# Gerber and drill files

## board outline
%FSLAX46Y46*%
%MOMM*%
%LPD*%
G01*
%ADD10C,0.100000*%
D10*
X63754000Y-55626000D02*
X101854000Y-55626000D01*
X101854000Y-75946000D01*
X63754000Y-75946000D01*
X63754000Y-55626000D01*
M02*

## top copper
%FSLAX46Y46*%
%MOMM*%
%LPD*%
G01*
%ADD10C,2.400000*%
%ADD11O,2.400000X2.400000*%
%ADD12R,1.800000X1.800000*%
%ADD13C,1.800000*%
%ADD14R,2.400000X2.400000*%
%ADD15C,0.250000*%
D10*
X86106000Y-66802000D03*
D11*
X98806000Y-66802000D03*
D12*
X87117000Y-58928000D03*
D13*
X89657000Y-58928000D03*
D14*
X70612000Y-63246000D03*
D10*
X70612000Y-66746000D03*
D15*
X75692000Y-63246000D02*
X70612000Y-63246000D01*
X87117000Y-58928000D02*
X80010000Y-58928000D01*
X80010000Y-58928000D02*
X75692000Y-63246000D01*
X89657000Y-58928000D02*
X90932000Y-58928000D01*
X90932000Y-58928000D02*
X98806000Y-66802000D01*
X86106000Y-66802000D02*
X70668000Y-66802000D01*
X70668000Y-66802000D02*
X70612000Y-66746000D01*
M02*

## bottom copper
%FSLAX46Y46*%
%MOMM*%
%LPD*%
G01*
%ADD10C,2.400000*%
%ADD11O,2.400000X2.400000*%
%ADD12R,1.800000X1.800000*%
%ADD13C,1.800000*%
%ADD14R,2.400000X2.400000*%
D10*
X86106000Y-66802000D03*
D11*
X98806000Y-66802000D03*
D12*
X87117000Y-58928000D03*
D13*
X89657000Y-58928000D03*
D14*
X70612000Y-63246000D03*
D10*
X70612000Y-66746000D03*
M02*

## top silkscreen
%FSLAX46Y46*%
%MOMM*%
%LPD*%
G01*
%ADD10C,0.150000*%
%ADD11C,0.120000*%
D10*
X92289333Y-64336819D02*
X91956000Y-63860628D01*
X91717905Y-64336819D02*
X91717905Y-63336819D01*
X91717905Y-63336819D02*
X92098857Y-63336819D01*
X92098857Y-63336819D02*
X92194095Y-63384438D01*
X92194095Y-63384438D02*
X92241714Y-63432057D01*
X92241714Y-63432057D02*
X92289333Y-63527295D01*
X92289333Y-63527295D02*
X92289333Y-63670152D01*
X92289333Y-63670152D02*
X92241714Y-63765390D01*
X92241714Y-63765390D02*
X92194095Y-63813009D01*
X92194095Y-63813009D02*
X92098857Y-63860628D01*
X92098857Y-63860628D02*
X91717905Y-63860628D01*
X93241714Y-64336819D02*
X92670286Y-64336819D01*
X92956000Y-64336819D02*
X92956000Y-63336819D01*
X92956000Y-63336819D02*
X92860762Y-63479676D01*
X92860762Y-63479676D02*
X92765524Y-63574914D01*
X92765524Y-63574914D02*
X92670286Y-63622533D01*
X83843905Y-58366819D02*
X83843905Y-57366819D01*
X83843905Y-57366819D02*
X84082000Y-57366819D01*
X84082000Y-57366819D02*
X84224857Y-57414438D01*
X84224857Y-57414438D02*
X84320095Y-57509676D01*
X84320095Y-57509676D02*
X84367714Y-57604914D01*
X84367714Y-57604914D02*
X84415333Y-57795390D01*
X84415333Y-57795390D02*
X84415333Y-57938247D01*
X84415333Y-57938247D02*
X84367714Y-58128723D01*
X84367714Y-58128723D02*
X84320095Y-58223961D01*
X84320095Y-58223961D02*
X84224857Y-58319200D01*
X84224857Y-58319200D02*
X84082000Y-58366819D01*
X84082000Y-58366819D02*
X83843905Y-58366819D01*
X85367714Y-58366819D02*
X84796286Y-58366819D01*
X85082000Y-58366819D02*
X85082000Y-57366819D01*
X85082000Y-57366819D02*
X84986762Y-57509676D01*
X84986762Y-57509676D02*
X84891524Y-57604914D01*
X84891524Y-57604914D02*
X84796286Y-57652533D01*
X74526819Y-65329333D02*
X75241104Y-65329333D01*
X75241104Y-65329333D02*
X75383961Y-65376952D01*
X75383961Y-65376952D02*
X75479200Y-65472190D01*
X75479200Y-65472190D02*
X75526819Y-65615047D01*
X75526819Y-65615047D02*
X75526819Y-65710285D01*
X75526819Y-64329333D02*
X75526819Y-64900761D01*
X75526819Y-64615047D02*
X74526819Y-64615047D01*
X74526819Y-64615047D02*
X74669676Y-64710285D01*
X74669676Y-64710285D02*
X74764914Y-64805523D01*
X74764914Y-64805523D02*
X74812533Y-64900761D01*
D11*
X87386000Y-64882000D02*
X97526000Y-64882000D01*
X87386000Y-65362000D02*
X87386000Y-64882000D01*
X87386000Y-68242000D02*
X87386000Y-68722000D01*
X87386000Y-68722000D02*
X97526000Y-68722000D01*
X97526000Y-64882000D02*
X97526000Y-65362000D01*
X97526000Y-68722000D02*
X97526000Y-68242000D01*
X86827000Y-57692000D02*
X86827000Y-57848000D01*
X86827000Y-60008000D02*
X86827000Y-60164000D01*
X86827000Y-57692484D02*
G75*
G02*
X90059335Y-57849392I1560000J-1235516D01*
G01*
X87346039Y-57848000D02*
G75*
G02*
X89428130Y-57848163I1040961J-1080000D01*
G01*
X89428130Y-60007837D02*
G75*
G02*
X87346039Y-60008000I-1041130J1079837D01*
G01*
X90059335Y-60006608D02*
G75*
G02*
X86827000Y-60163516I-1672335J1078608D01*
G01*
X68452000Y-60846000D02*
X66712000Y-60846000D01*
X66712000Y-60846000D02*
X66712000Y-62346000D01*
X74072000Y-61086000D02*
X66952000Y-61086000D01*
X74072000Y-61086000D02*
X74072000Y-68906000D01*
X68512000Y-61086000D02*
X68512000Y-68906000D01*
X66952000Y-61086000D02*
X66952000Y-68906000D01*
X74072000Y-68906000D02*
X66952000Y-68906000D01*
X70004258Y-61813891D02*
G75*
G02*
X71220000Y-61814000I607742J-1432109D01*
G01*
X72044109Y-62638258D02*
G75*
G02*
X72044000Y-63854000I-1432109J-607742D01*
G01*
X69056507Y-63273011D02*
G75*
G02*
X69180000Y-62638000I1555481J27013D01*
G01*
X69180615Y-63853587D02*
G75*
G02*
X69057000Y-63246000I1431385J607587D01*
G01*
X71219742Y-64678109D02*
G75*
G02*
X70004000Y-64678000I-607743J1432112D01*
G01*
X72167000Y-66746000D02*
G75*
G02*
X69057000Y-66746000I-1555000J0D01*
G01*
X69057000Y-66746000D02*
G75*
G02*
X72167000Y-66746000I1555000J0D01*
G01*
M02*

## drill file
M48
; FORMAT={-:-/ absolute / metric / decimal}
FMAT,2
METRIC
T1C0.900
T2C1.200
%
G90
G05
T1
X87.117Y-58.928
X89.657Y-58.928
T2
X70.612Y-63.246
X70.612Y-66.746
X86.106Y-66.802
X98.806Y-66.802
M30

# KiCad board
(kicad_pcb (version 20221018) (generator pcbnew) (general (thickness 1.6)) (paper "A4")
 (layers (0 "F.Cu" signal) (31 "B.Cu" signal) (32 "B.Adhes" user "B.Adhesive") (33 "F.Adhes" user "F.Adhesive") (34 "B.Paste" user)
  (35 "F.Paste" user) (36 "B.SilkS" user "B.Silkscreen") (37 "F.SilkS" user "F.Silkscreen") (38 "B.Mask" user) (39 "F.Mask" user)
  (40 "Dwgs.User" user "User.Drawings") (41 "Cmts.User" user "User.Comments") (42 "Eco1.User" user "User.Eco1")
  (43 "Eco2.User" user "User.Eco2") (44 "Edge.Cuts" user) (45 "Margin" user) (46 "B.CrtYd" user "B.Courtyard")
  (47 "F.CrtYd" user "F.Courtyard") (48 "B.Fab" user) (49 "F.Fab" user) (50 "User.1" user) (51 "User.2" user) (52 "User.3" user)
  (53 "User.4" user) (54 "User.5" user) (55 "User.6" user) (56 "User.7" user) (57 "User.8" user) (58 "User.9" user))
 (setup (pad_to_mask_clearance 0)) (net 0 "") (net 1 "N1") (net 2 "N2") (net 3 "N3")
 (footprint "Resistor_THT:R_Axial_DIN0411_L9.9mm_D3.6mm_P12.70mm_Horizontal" (layer "F.Cu") (at 86.106 66.802)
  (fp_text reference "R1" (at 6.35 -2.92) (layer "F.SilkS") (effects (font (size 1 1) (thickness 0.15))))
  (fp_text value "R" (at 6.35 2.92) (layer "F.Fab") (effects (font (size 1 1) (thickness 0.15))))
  (fp_line (start 1.28 -1.92) (end 11.42 -1.92) (stroke (width 0.12) (type solid)) (layer "F.SilkS"))
  (fp_line (start 1.28 -1.44) (end 1.28 -1.92) (stroke (width 0.12) (type solid)) (layer "F.SilkS"))
  (fp_line (start 1.28 1.44) (end 1.28 1.92) (stroke (width 0.12) (type solid)) (layer "F.SilkS"))
  (fp_line (start 1.28 1.92) (end 11.42 1.92) (stroke (width 0.12) (type solid)) (layer "F.SilkS"))
  (fp_line (start 11.42 -1.92) (end 11.42 -1.44) (stroke (width 0.12) (type solid)) (layer "F.SilkS"))
  (fp_line (start 11.42 1.92) (end 11.42 1.44) (stroke (width 0.12) (type solid)) (layer "F.SilkS"))
  (pad "1" thru_hole circle (at 0 0) (size 2.4 2.4) (drill 1.2) (layers "*.Cu" "*.Mask") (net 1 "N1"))
  (pad "2" thru_hole oval (at 12.7 0) (size 2.4 2.4) (drill 1.2) (layers "*.Cu" "*.Mask") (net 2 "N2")))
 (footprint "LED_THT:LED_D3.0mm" (layer "F.Cu") (at 87.117 58.928)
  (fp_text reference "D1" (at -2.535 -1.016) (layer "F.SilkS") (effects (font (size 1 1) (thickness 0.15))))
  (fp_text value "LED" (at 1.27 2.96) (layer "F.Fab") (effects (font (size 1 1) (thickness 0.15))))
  (fp_line (start -0.29 -1.236) (end -0.29 -1.08) (stroke (width 0.12) (type solid)) (layer "F.SilkS"))
  (fp_line (start -0.29 1.08) (end -0.29 1.236) (stroke (width 0.12) (type solid)) (layer "F.SilkS"))
  (fp_arc (start -0.29 -1.235516) (mid 1.366487 -1.987659) (end 2.942335 -1.078608) (stroke (width 0.12) (type solid)) (layer "F.SilkS"))
  (fp_arc (start 0.229039 -1.08) (mid 1.270117 -1.5) (end 2.31113 -1.079837) (stroke (width 0.12) (type solid)) (layer "F.SilkS"))
  (fp_arc (start 2.31113 1.079837) (mid 1.270117 1.5) (end 0.229039 1.08) (stroke (width 0.12) (type solid)) (layer "F.SilkS"))
  (fp_arc (start 2.942335 1.078608) (mid 1.366487 1.987659) (end -0.29 1.235516) (stroke (width 0.12) (type solid)) (layer "F.SilkS"))
  (pad "1" thru_hole rect (at 0 0) (size 1.8 1.8) (drill 0.9) (layers "*.Cu" "*.Mask") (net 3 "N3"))
  (pad "2" thru_hole circle (at 2.54 0) (size 1.8 1.8) (drill 0.9) (layers "*.Cu" "*.Mask") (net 2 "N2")))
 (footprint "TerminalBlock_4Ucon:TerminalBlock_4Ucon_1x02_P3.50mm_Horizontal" (layer "F.Cu") (at 70.612 63.246 -90)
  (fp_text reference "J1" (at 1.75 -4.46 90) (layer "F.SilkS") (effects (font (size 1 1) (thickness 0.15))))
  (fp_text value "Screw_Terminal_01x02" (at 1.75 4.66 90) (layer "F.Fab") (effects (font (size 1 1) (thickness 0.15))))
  (fp_line (start -2.4 2.16) (end -2.4 3.9) (stroke (width 0.12) (type solid)) (layer "F.SilkS"))
  (fp_line (start -2.4 3.9) (end -0.9 3.9) (stroke (width 0.12) (type solid)) (layer "F.SilkS"))
  (fp_line (start -2.16 -3.46) (end -2.16 3.66) (stroke (width 0.12) (type solid)) (layer "F.SilkS"))
  (fp_line (start -2.16 -3.46) (end 5.66 -3.46) (stroke (width 0.12) (type solid)) (layer "F.SilkS"))
  (fp_line (start -2.16 2.1) (end 5.66 2.1) (stroke (width 0.12) (type solid)) (layer "F.SilkS"))
  (fp_line (start -2.16 3.66) (end 5.66 3.66) (stroke (width 0.12) (type solid)) (layer "F.SilkS"))
  (fp_line (start 5.66 -3.46) (end 5.66 3.66) (stroke (width 0.12) (type solid)) (layer "F.SilkS"))
  (fp_arc (start -1.432109 0.607742) (mid -1.555727 -0.00014) (end -1.432 -0.608) (stroke (width 0.12) (type solid)) (layer "F.SilkS"))
  (fp_arc (start -0.607742 -1.432109) (mid 0.00014 -1.555727) (end 0.608 -1.432) (stroke (width 0.12) (type solid)) (layer "F.SilkS"))
  (fp_arc (start 0.027011 1.555493) (mid -0.296984 1.527118) (end -0.608 1.432) (stroke (width 0.12) (type solid)) (layer "F.SilkS"))
  (fp_arc (start 0.607587 1.431385) (mid 0.310017 1.523783) (end 0 1.555) (stroke (width 0.12) (type solid)) (layer "F.SilkS"))
  (fp_arc (start 1.432109 -0.607742) (mid 1.555727 0.00014) (end 1.432 0.608) (stroke (width 0.12) (type solid)) (layer "F.SilkS"))
  (fp_circle (center 3.5 0) (end 5.055 0) (stroke (width 0.12) (type solid)) (fill none) (layer "F.SilkS"))
  (pad "1" thru_hole rect (at 0 0 270) (size 2.4 2.4) (drill 1.2) (layers "*.Cu" "*.Mask") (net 3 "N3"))
  (pad "2" thru_hole circle (at 3.5 0 270) (size 2.4 2.4) (drill 1.2) (layers "*.Cu" "*.Mask") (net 1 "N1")))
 (gr_rect (start 63.754 55.626) (end 101.854 75.946) (stroke (width 0.1) (type default)) (fill none) (layer "Edge.Cuts"))
 (segment (start 75.692 63.246) (end 70.612 63.246) (width 0.25) (layer "F.Cu") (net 3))
 (segment (start 87.117 58.928) (end 80.01 58.928) (width 0.25) (layer "F.Cu") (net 3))
 (segment (start 80.01 58.928) (end 75.692 63.246) (width 0.25) (layer "F.Cu") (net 3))
 (segment (start 89.657 58.928) (end 90.932 58.928) (width 0.25) (layer "F.Cu") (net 2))
 (segment (start 90.932 58.928) (end 98.806 66.802) (width 0.25) (layer "F.Cu") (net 2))
 (segment (start 86.106 66.802) (end 70.668 66.802) (width 0.25) (layer "F.Cu") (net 1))
 (segment (start 70.668 66.802) (end 70.612 66.746) (width 0.25) (layer "F.Cu") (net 1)))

